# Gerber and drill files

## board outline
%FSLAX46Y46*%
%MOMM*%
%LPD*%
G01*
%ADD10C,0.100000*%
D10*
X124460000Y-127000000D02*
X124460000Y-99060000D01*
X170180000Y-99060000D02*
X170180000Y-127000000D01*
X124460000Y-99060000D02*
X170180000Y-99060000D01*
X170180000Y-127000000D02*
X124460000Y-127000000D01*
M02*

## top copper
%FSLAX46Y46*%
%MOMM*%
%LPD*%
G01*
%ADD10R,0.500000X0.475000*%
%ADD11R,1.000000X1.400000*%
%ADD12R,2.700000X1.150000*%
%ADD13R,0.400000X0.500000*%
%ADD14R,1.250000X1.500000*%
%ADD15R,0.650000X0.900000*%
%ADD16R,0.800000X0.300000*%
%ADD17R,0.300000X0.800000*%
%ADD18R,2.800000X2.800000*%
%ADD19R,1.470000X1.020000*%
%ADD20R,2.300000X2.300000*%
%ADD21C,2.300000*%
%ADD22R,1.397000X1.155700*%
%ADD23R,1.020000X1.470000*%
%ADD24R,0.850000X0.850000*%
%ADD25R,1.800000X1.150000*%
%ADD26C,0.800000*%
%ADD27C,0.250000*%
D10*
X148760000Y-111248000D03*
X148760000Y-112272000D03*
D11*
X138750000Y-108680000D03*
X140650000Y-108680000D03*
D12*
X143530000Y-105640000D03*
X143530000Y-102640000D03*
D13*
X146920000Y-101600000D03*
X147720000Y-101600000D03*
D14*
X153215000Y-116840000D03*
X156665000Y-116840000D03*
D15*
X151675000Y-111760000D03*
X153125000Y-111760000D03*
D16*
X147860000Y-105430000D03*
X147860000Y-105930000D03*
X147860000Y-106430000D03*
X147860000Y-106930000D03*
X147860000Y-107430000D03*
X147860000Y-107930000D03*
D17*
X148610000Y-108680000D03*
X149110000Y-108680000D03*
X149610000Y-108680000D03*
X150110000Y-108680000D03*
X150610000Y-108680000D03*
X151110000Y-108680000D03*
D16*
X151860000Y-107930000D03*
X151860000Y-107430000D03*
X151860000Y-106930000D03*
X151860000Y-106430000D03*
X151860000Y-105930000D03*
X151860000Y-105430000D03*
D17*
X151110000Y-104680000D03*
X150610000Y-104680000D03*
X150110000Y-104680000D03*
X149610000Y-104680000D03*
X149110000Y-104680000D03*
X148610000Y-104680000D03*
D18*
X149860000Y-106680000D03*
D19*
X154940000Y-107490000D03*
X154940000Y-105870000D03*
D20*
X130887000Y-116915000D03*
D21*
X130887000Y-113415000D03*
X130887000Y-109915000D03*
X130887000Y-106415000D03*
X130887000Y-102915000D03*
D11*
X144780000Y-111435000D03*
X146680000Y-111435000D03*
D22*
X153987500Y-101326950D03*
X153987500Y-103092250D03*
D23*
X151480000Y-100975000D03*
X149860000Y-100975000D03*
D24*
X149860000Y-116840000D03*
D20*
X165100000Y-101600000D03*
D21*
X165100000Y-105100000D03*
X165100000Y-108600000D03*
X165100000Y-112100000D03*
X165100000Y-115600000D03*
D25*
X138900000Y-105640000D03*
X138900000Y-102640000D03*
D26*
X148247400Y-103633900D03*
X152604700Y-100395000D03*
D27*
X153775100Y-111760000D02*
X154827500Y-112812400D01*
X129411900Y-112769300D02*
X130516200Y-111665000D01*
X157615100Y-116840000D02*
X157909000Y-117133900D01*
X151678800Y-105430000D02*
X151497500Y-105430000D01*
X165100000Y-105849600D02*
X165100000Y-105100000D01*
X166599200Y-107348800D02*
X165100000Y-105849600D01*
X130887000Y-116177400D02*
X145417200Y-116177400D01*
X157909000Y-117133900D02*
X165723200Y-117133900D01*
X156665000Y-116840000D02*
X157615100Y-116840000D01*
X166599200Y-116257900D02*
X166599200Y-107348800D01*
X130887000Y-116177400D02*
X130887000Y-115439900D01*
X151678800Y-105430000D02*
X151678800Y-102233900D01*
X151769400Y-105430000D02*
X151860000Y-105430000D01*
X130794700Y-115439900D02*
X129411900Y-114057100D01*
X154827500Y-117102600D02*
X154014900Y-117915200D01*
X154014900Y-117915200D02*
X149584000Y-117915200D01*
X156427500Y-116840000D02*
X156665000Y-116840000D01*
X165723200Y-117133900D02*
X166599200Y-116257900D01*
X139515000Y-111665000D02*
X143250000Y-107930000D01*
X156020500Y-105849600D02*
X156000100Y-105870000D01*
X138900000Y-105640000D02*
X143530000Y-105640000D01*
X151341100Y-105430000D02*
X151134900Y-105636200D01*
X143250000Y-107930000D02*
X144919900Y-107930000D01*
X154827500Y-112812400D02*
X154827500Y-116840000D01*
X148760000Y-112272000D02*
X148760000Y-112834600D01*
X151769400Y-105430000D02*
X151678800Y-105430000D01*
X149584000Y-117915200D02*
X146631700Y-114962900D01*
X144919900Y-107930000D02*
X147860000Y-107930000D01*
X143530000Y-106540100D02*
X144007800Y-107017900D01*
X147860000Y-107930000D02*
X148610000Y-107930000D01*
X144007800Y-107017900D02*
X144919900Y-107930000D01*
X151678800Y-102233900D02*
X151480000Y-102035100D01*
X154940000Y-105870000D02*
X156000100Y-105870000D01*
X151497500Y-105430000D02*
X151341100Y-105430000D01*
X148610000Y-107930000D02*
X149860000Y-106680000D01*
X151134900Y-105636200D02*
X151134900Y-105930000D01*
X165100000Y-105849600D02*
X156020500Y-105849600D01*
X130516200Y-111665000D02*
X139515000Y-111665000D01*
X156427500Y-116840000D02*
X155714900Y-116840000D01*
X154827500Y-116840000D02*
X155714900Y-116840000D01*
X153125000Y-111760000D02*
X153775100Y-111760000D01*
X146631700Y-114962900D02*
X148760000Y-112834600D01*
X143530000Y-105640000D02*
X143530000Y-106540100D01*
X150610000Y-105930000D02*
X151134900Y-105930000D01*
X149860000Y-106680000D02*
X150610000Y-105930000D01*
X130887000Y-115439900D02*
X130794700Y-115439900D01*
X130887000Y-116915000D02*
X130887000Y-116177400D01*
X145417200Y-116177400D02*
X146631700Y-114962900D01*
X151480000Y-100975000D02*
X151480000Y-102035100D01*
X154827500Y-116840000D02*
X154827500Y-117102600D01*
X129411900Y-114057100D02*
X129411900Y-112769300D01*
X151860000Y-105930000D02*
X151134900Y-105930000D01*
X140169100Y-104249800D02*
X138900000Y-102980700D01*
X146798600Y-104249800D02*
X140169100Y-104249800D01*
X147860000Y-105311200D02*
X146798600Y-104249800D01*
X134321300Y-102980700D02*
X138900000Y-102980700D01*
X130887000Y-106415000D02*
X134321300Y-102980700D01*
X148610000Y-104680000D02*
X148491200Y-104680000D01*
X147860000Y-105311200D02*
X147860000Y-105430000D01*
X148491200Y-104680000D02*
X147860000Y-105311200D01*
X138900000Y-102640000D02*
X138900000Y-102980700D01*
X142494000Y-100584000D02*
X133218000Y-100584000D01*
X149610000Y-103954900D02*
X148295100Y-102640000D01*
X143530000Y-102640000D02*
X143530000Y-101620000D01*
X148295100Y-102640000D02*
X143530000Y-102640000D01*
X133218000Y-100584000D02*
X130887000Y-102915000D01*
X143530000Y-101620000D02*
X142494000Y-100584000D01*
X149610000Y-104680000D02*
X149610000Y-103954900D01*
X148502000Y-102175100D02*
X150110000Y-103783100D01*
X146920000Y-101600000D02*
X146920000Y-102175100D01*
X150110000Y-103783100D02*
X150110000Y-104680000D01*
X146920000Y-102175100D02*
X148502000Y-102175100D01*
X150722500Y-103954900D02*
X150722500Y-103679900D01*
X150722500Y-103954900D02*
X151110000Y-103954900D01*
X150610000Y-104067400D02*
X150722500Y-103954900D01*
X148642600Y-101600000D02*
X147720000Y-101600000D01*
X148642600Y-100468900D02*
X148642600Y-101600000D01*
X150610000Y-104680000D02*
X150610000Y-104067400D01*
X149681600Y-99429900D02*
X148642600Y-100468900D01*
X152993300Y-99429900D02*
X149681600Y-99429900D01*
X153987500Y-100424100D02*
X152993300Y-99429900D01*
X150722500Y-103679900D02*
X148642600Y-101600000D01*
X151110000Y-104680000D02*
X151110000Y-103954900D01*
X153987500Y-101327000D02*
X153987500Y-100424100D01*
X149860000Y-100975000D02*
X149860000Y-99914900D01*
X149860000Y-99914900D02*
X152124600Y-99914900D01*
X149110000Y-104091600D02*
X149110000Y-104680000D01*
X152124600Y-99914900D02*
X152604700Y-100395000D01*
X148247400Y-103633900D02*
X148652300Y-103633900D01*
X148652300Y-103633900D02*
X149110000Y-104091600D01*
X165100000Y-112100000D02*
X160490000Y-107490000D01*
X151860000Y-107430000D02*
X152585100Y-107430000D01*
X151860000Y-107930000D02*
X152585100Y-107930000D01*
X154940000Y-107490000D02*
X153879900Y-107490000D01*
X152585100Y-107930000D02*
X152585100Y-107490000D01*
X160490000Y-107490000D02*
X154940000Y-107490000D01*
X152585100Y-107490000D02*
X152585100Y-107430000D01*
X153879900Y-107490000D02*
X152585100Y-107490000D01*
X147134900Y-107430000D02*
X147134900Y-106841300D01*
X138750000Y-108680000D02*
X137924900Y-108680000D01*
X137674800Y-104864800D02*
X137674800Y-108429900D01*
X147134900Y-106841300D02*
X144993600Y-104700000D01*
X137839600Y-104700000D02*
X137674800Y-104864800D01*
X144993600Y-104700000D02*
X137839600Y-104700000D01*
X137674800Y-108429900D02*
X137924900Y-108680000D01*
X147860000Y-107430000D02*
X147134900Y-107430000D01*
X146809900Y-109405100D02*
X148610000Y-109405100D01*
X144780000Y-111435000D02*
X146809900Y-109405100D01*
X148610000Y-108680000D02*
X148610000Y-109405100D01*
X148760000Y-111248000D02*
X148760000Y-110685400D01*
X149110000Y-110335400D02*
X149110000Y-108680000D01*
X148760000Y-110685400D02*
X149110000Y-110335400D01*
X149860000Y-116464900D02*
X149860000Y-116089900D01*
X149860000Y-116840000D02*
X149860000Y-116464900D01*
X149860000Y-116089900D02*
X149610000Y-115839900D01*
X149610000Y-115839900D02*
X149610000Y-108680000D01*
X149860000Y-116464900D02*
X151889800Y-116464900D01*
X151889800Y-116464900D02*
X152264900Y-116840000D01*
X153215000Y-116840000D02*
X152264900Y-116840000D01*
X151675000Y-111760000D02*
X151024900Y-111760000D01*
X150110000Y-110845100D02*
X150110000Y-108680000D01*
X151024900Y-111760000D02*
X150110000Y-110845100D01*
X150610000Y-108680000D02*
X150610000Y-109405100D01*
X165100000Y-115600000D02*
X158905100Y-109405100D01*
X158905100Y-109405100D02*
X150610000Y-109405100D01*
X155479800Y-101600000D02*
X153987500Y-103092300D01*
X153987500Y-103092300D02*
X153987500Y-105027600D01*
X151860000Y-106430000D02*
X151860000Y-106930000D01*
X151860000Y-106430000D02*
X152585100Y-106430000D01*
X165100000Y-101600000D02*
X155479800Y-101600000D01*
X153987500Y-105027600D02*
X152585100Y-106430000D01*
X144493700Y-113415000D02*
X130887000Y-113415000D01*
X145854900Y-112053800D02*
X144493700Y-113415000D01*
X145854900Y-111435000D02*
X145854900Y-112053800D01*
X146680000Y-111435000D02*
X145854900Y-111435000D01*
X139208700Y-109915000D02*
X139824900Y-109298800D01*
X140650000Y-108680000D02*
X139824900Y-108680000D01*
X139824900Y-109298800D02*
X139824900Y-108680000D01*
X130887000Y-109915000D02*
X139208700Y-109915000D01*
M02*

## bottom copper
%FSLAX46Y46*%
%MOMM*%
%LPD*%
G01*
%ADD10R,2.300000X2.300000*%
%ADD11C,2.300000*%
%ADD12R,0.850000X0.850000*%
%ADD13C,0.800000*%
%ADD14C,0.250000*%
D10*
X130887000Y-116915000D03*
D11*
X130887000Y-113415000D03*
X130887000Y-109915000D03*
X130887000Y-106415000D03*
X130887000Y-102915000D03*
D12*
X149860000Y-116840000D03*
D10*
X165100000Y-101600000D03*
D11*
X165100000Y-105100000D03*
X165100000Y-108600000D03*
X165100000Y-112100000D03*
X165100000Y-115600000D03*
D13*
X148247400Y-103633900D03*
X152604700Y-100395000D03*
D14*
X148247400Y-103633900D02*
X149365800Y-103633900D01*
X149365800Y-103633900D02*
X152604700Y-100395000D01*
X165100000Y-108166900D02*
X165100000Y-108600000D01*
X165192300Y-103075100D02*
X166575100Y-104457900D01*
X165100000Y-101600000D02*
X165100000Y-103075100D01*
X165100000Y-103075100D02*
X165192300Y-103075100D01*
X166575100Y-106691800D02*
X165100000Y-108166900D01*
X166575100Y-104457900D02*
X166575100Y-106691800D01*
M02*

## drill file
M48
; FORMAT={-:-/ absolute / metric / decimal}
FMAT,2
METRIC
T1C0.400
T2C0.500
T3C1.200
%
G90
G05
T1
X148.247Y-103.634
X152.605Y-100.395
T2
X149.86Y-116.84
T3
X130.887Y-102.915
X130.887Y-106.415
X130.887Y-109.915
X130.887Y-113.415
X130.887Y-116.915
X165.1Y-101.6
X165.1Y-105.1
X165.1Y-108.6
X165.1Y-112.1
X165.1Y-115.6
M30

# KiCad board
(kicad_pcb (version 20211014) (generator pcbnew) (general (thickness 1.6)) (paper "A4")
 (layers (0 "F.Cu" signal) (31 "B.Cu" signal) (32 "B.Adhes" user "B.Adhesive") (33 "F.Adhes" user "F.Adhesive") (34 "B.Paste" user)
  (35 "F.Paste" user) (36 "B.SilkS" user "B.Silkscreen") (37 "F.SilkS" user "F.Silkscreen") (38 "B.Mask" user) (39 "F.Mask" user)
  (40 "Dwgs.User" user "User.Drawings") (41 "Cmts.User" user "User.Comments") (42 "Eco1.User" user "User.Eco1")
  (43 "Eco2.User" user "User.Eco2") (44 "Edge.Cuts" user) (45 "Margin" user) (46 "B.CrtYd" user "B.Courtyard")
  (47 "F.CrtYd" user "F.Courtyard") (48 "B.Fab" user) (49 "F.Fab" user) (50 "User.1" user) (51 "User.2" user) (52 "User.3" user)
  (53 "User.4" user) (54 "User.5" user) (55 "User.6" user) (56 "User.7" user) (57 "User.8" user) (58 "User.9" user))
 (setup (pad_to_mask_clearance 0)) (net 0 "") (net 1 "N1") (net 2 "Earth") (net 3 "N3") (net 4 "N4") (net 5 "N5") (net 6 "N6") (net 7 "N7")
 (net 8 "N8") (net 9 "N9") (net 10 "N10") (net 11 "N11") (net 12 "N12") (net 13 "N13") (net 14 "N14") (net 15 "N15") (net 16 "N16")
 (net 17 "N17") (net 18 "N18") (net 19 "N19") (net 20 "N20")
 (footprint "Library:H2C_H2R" (layer "F.Cu") (at 148.76 111.76 -90)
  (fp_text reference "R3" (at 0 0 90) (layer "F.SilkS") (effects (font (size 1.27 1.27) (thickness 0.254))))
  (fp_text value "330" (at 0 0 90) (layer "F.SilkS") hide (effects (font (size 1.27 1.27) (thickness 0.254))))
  (pad "1" smd rect locked (at -0.512 0 270) (size 0.475 0.5) (layers "F.Cu" "F.Paste" "F.Mask") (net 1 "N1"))
  (pad "2" smd rect locked (at 0.512 0 270) (size 0.475 0.5) (layers "F.Cu" "F.Paste" "F.Mask") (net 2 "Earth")))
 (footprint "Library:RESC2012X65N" (layer "F.Cu") (at 139.7 108.68)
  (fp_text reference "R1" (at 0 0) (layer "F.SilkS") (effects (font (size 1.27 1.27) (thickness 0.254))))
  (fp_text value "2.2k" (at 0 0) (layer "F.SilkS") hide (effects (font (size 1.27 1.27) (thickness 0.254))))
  (pad "1" smd rect (at -0.95 0) (size 1 1.4) (layers "F.Cu" "F.Paste" "F.Mask") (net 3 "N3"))
  (pad "2" smd rect (at 0.95 0) (size 1 1.4) (layers "F.Cu" "F.Paste" "F.Mask") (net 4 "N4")))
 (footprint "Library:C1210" (layer "F.Cu") (at 143.53 104.14 90)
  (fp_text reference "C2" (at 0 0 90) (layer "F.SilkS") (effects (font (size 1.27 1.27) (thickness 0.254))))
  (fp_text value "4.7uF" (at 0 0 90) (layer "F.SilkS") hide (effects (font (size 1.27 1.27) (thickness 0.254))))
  (pad "1" smd rect (at -1.5 0 90) (size 1.15 2.7) (layers "F.Cu" "F.Paste" "F.Mask") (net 2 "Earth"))
  (pad "2" smd rect (at 1.5 0 90) (size 1.15 2.7) (layers "F.Cu" "F.Paste" "F.Mask") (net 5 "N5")))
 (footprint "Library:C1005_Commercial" (layer "F.Cu") (at 147.32 101.6)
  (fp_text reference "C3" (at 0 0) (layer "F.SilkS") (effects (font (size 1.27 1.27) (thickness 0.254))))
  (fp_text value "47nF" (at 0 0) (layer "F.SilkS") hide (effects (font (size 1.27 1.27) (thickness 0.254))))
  (pad "1" smd rect (at -0.4 0) (size 0.4 0.5) (layers "F.Cu" "F.Paste" "F.Mask") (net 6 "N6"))
  (pad "2" smd rect (at 0.4 0) (size 0.4 0.5) (layers "F.Cu" "F.Paste" "F.Mask") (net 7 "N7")))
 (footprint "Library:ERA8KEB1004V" (layer "F.Cu") (at 154.94 116.84)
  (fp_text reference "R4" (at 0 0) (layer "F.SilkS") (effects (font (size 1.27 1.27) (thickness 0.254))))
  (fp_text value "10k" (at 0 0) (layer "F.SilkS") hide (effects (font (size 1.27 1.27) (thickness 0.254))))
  (pad "1" smd rect locked (at -1.725 0) (size 1.25 1.5) (layers "F.Cu" "F.Paste" "F.Mask") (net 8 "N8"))
  (pad "2" smd rect locked (at 1.725 0) (size 1.25 1.5) (layers "F.Cu" "F.Paste" "F.Mask") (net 2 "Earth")))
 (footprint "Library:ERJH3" (layer "F.Cu") (at 152.4 111.76)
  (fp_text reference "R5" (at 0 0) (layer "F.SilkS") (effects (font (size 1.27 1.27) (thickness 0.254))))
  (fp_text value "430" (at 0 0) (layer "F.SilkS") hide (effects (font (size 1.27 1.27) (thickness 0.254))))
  (pad "1" smd rect locked (at -0.725 0) (size 0.65 0.9) (layers "F.Cu" "F.Paste" "F.Mask") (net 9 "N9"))
  (pad "2" smd rect locked (at 0.725 0) (size 0.65 0.9) (layers "F.Cu" "F.Paste" "F.Mask") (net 2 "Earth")))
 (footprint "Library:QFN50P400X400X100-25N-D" (layer "F.Cu") (at 149.86 106.68)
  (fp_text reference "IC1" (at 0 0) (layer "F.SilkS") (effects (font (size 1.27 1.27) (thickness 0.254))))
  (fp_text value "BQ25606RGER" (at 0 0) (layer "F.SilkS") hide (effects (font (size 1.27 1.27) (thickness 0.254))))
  (pad "1" smd rect (at -2 -1.25 90) (size 0.3 0.8) (layers "F.Cu" "F.Paste" "F.Mask") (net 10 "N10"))
  (pad "2" smd rect (at -2 -0.75 90) (size 0.3 0.8) (layers "F.Cu" "F.Paste" "F.Mask") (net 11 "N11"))
  (pad "3" smd rect (at -2 -0.25 90) (size 0.3 0.8) (layers "F.Cu" "F.Paste" "F.Mask") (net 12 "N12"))
  (pad "4" smd rect (at -2 0.25 90) (size 0.3 0.8) (layers "F.Cu" "F.Paste" "F.Mask") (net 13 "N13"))
  (pad "5" smd rect (at -2 0.75 90) (size 0.3 0.8) (layers "F.Cu" "F.Paste" "F.Mask") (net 3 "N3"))
  (pad "6" smd rect (at -2 1.25 90) (size 0.3 0.8) (layers "F.Cu" "F.Paste" "F.Mask") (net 2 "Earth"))
  (pad "7" smd rect (at -1.25 2) (size 0.3 0.8) (layers "F.Cu" "F.Paste" "F.Mask") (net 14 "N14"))
  (pad "8" smd rect (at -0.75 2) (size 0.3 0.8) (layers "F.Cu" "F.Paste" "F.Mask") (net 1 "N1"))
  (pad "9" smd rect (at -0.25 2) (size 0.3 0.8) (layers "F.Cu" "F.Paste" "F.Mask") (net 8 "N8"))
  (pad "10" smd rect (at 0.25 2) (size 0.3 0.8) (layers "F.Cu" "F.Paste" "F.Mask") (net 9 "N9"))
  (pad "11" smd rect (at 0.75 2) (size 0.3 0.8) (layers "F.Cu" "F.Paste" "F.Mask") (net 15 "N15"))
  (pad "12" smd rect (at 1.25 2) (size 0.3 0.8) (layers "F.Cu" "F.Paste" "F.Mask") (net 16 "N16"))
  (pad "13" smd rect (at 2 1.25 90) (size 0.3 0.8) (layers "F.Cu" "F.Paste" "F.Mask") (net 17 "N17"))
  (pad "14" smd rect (at 2 0.75 90) (size 0.3 0.8) (layers "F.Cu" "F.Paste" "F.Mask") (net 17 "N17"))
  (pad "15" smd rect (at 2 0.25 90) (size 0.3 0.8) (layers "F.Cu" "F.Paste" "F.Mask") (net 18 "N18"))
  (pad "16" smd rect (at 2 -0.25 90) (size 0.3 0.8) (layers "F.Cu" "F.Paste" "F.Mask") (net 18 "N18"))
  (pad "17" smd rect (at 2 -0.75 90) (size 0.3 0.8) (layers "F.Cu" "F.Paste" "F.Mask") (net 2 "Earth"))
  (pad "18" smd rect (at 2 -1.25 90) (size 0.3 0.8) (layers "F.Cu" "F.Paste" "F.Mask") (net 2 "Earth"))
  (pad "19" smd rect (at 1.25 -2) (size 0.3 0.8) (layers "F.Cu" "F.Paste" "F.Mask") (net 7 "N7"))
  (pad "20" smd rect (at 0.75 -2) (size 0.3 0.8) (layers "F.Cu" "F.Paste" "F.Mask") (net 7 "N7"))
  (pad "21" smd rect (at 0.25 -2) (size 0.3 0.8) (layers "F.Cu" "F.Paste" "F.Mask") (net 6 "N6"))
  (pad "22" smd rect (at -0.25 -2) (size 0.3 0.8) (layers "F.Cu" "F.Paste" "F.Mask") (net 5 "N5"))
  (pad "23" smd rect (at -0.75 -2) (size 0.3 0.8) (layers "F.Cu" "F.Paste" "F.Mask") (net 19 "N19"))
  (pad "24" smd rect (at -1.25 -2) (size 0.3 0.8) (layers "F.Cu" "F.Paste" "F.Mask") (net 10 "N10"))
  (pad "25" smd rect (at 0 0) (size 2.8 2.8) (layers "F.Cu" "F.Paste" "F.Mask") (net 2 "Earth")))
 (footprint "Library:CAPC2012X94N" (layer "F.Cu") (at 154.94 106.68 90)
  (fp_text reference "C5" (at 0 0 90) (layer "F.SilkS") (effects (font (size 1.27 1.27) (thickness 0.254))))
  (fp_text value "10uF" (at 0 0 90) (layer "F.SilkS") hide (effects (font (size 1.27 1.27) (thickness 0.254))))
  (pad "1" smd rect (at -0.81 0 90) (size 1.02 1.47) (layers "F.Cu" "F.Paste" "F.Mask") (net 17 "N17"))
  (pad "2" smd rect (at 0.81 0 90) (size 1.02 1.47) (layers "F.Cu" "F.Paste" "F.Mask") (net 2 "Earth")))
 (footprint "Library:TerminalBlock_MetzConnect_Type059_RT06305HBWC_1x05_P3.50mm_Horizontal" (layer "F.Cu") (at 130.887 116.915 90)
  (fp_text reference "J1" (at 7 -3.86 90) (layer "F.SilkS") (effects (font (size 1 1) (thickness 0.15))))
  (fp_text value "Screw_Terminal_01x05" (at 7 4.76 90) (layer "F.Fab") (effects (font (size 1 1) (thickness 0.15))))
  (pad "1" thru_hole rect (at 0 0 90) (size 2.3 2.3) (drill 1.2) (layers *.Cu *.Mask) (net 2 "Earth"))
  (pad "2" thru_hole circle (at 3.5 0 90) (size 2.3 2.3) (drill 1.2) (layers *.Cu *.Mask) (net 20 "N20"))
  (pad "3" thru_hole circle (at 7 0 90) (size 2.3 2.3) (drill 1.2) (layers *.Cu *.Mask) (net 4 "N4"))
  (pad "4" thru_hole circle (at 10.5 0 90) (size 2.3 2.3) (drill 1.2) (layers *.Cu *.Mask) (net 10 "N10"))
  (pad "5" thru_hole circle (at 14 0 90) (size 2.3 2.3) (drill 1.2) (layers *.Cu *.Mask) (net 5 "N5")))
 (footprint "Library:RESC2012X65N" (layer "F.Cu") (at 145.73 111.435)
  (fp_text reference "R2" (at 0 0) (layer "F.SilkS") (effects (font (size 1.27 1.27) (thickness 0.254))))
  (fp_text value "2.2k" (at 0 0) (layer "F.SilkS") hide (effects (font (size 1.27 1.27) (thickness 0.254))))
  (pad "1" smd rect (at -0.95 0) (size 1 1.4) (layers "F.Cu" "F.Paste" "F.Mask") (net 14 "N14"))
  (pad "2" smd rect (at 0.95 0) (size 1 1.4) (layers "F.Cu" "F.Paste" "F.Mask") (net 20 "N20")))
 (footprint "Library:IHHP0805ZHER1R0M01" (layer "F.Cu") (at 153.9875 102.2096 -90)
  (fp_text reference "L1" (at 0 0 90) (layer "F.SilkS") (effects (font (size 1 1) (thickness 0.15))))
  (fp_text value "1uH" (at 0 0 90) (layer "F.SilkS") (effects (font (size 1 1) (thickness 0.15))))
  (pad "1" smd rect (at -0.88265 0 270) (size 1.1557 1.397) (layers "F.Cu" "F.Paste" "F.Mask") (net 7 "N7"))
  (pad "2" smd rect (at 0.88265 0 270) (size 1.1557 1.397) (layers "F.Cu" "F.Paste" "F.Mask") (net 18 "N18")))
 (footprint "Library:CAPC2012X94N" (layer "F.Cu") (at 150.67 100.975 180)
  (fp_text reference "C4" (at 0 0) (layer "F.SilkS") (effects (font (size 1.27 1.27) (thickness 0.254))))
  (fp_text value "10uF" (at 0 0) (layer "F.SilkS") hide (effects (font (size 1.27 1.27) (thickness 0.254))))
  (pad "1" smd rect (at -0.81 0 180) (size 1.02 1.47) (layers "F.Cu" "F.Paste" "F.Mask") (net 2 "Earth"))
  (pad "2" smd rect (at 0.81 0 180) (size 1.02 1.47) (layers "F.Cu" "F.Paste" "F.Mask") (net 19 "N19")))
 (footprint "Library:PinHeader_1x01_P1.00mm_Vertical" (layer "F.Cu") (at 149.86 116.84)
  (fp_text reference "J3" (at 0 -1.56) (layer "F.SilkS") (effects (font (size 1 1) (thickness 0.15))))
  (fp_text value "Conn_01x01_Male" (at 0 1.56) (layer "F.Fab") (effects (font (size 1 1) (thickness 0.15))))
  (pad "1" thru_hole rect (at 0 0) (size 0.85 0.85) (drill 0.5) (layers *.Cu *.Mask) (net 8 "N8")))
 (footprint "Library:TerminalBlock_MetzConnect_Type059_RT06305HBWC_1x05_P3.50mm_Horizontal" (layer "F.Cu") (at 165.1 101.6 -90)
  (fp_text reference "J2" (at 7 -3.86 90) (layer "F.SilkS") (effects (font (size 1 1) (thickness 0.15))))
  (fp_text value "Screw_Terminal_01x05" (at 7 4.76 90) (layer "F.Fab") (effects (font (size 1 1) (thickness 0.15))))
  (pad "1" thru_hole rect (at 0 0 270) (size 2.3 2.3) (drill 1.2) (layers *.Cu *.Mask) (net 18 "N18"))
  (pad "2" thru_hole circle (at 3.5 0 270) (size 2.3 2.3) (drill 1.2) (layers *.Cu *.Mask) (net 2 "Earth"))
  (pad "3" thru_hole circle (at 7 0 270) (size 2.3 2.3) (drill 1.2) (layers *.Cu *.Mask) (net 18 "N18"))
  (pad "4" thru_hole circle (at 10.5 0 270) (size 2.3 2.3) (drill 1.2) (layers *.Cu *.Mask) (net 17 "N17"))
  (pad "5" thru_hole circle (at 14 0 270) (size 2.3 2.3) (drill 1.2) (layers *.Cu *.Mask) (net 15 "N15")))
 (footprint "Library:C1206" (layer "F.Cu") (at 138.9 104.14 90)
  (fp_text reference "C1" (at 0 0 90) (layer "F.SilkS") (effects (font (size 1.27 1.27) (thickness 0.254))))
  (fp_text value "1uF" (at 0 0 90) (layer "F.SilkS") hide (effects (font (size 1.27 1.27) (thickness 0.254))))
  (pad "1" smd rect (at -1.5 0 90) (size 1.15 1.8) (layers "F.Cu" "F.Paste" "F.Mask") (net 2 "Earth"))
  (pad "2" smd rect (at 1.5 0 90) (size 1.15 1.8) (layers "F.Cu" "F.Paste" "F.Mask") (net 10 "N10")))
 (gr_line (start 124.46 127) (end 124.46 99.06) (layer "Edge.Cuts") (width 0.1))
 (gr_line (start 170.18 99.06) (end 170.18 127) (layer "Edge.Cuts") (width 0.1))
 (gr_line (start 124.46 99.06) (end 170.18 99.06) (layer "Edge.Cuts") (width 0.1))
 (gr_line (start 170.18 127) (end 124.46 127) (layer "Edge.Cuts") (width 0.1))
 (segment (start 153.7751 111.76) (end 154.8275 112.8124) (width 0.25) (layer "F.Cu") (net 2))
 (segment (start 129.4119 112.7693) (end 130.5162 111.665) (width 0.25) (layer "F.Cu") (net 2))
 (segment (start 157.6151 116.84) (end 157.909 117.1339) (width 0.25) (layer "F.Cu") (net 2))
 (segment (start 151.6788 105.43) (end 151.4975 105.43) (width 0.25) (layer "F.Cu") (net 2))
 (segment (start 165.1 105.8496) (end 165.1 105.1) (width 0.25) (layer "F.Cu") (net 2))
 (segment (start 166.5992 107.3488) (end 165.1 105.8496) (width 0.25) (layer "F.Cu") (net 2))
 (segment (start 130.887 116.1774) (end 145.4172 116.1774) (width 0.25) (layer "F.Cu") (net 2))
 (segment (start 157.909 117.1339) (end 165.7232 117.1339) (width 0.25) (layer "F.Cu") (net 2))
 (segment (start 156.665 116.84) (end 157.6151 116.84) (width 0.25) (layer "F.Cu") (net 2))
 (segment (start 166.5992 116.2579) (end 166.5992 107.3488) (width 0.25) (layer "F.Cu") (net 2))
 (segment (start 130.887 116.1774) (end 130.887 115.4399) (width 0.25) (layer "F.Cu") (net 2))
 (segment (start 151.6788 105.43) (end 151.6788 102.2339) (width 0.25) (layer "F.Cu") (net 2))
 (segment (start 151.7694 105.43) (end 151.86 105.43) (width 0.25) (layer "F.Cu") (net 2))
 (segment (start 130.7947 115.4399) (end 129.4119 114.0571) (width 0.25) (layer "F.Cu") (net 2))
 (segment (start 154.8275 117.1026) (end 154.0149 117.9152) (width 0.25) (layer "F.Cu") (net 2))
 (segment (start 154.0149 117.9152) (end 149.584 117.9152) (width 0.25) (layer "F.Cu") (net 2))
 (segment (start 156.4275 116.84) (end 156.665 116.84) (width 0.25) (layer "F.Cu") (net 2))
 (segment (start 165.7232 117.1339) (end 166.5992 116.2579) (width 0.25) (layer "F.Cu") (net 2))
 (segment (start 139.515 111.665) (end 143.25 107.93) (width 0.25) (layer "F.Cu") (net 2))
 (segment (start 156.0205 105.8496) (end 156.0001 105.87) (width 0.25) (layer "F.Cu") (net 2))
 (segment (start 138.9 105.64) (end 143.53 105.64) (width 0.25) (layer "F.Cu") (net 2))
 (segment (start 151.3411 105.43) (end 151.1349 105.6362) (width 0.25) (layer "F.Cu") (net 2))
 (segment (start 143.25 107.93) (end 144.9199 107.93) (width 0.25) (layer "F.Cu") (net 2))
 (segment (start 154.8275 112.8124) (end 154.8275 116.84) (width 0.25) (layer "F.Cu") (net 2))
 (segment (start 148.76 112.272) (end 148.76 112.8346) (width 0.25) (layer "F.Cu") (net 2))
 (segment (start 151.7694 105.43) (end 151.6788 105.43) (width 0.25) (layer "F.Cu") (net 2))
 (segment (start 149.584 117.9152) (end 146.6317 114.9629) (width 0.25) (layer "F.Cu") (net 2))
 (segment (start 144.9199 107.93) (end 147.86 107.93) (width 0.25) (layer "F.Cu") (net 2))
 (segment (start 143.53 106.5401) (end 144.0078 107.0179) (width 0.25) (layer "F.Cu") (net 2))
 (segment (start 147.86 107.93) (end 148.61 107.93) (width 0.25) (layer "F.Cu") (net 2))
 (segment (start 144.0078 107.0179) (end 144.9199 107.93) (width 0.25) (layer "F.Cu") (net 2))
 (segment (start 151.6788 102.2339) (end 151.48 102.0351) (width 0.25) (layer "F.Cu") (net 2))
 (segment (start 154.94 105.87) (end 156.0001 105.87) (width 0.25) (layer "F.Cu") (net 2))
 (segment (start 151.4975 105.43) (end 151.3411 105.43) (width 0.25) (layer "F.Cu") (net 2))
 (segment (start 148.61 107.93) (end 149.86 106.68) (width 0.25) (layer "F.Cu") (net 2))
 (segment (start 151.1349 105.6362) (end 151.1349 105.93) (width 0.25) (layer "F.Cu") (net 2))
 (segment (start 165.1 105.8496) (end 156.0205 105.8496) (width 0.25) (layer "F.Cu") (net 2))
 (segment (start 130.5162 111.665) (end 139.515 111.665) (width 0.25) (layer "F.Cu") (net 2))
 (segment (start 156.4275 116.84) (end 155.7149 116.84) (width 0.25) (layer "F.Cu") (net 2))
 (segment (start 154.8275 116.84) (end 155.7149 116.84) (width 0.25) (layer "F.Cu") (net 2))
 (segment (start 153.125 111.76) (end 153.7751 111.76) (width 0.25) (layer "F.Cu") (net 2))
 (segment (start 146.6317 114.9629) (end 148.76 112.8346) (width 0.25) (layer "F.Cu") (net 2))
 (segment (start 143.53 105.64) (end 143.53 106.5401) (width 0.25) (layer "F.Cu") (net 2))
 (segment (start 150.61 105.93) (end 151.1349 105.93) (width 0.25) (layer "F.Cu") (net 2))
 (segment (start 149.86 106.68) (end 150.61 105.93) (width 0.25) (layer "F.Cu") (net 2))
 (segment (start 130.887 115.4399) (end 130.7947 115.4399) (width 0.25) (layer "F.Cu") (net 2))
 (segment (start 130.887 116.915) (end 130.887 116.1774) (width 0.25) (layer "F.Cu") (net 2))
 (segment (start 145.4172 116.1774) (end 146.6317 114.9629) (width 0.25) (layer "F.Cu") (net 2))
 (segment (start 151.48 100.975) (end 151.48 102.0351) (width 0.25) (layer "F.Cu") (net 2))
 (segment (start 154.8275 116.84) (end 154.8275 117.1026) (width 0.25) (layer "F.Cu") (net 2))
 (segment (start 129.4119 114.0571) (end 129.4119 112.7693) (width 0.25) (layer "F.Cu") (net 2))
 (segment (start 151.86 105.93) (end 151.1349 105.93) (width 0.25) (layer "F.Cu") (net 2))
 (segment (start 140.1691 104.2498) (end 138.9 102.9807) (width 0.25) (layer "F.Cu") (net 10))
 (segment (start 146.7986 104.2498) (end 140.1691 104.2498) (width 0.25) (layer "F.Cu") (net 10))
 (segment (start 147.86 105.3112) (end 146.7986 104.2498) (width 0.25) (layer "F.Cu") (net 10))
 (segment (start 134.3213 102.9807) (end 138.9 102.9807) (width 0.25) (layer "F.Cu") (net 10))
 (segment (start 130.887 106.415) (end 134.3213 102.9807) (width 0.25) (layer "F.Cu") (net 10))
 (segment (start 148.61 104.68) (end 148.4912 104.68) (width 0.25) (layer "F.Cu") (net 10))
 (segment (start 147.86 105.3112) (end 147.86 105.43) (width 0.25) (layer "F.Cu") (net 10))
 (segment (start 148.4912 104.68) (end 147.86 105.3112) (width 0.25) (layer "F.Cu") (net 10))
 (segment (start 138.9 102.64) (end 138.9 102.9807) (width 0.25) (layer "F.Cu") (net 10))
 (segment (start 142.494 100.584) (end 133.218 100.584) (width 0.25) (layer "F.Cu") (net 5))
 (segment (start 149.61 103.9549) (end 148.2951 102.64) (width 0.25) (layer "F.Cu") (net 5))
 (segment (start 143.53 102.64) (end 143.53 101.62) (width 0.25) (layer "F.Cu") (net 5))
 (segment (start 148.2951 102.64) (end 143.53 102.64) (width 0.25) (layer "F.Cu") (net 5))
 (segment (start 133.218 100.584) (end 130.887 102.915) (width 0.25) (layer "F.Cu") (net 5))
 (segment (start 143.53 101.62) (end 142.494 100.584) (width 0.25) (layer "F.Cu") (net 5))
 (segment (start 149.61 104.68) (end 149.61 103.9549) (width 0.25) (layer "F.Cu") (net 5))
 (segment (start 148.502 102.1751) (end 150.11 103.7831) (width 0.25) (layer "F.Cu") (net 6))
 (segment (start 146.92 101.6) (end 146.92 102.1751) (width 0.25) (layer "F.Cu") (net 6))
 (segment (start 150.11 103.7831) (end 150.11 104.68) (width 0.25) (layer "F.Cu") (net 6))
 (segment (start 146.92 102.1751) (end 148.502 102.1751) (width 0.25) (layer "F.Cu") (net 6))
 (segment (start 150.7225 103.9549) (end 150.7225 103.6799) (width 0.25) (layer "F.Cu") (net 7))
 (segment (start 150.7225 103.9549) (end 151.11 103.9549) (width 0.25) (layer "F.Cu") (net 7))
 (segment (start 150.61 104.0674) (end 150.7225 103.9549) (width 0.25) (layer "F.Cu") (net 7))
 (segment (start 148.6426 101.6) (end 147.72 101.6) (width 0.25) (layer "F.Cu") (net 7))
 (segment (start 148.6426 100.4689) (end 148.6426 101.6) (width 0.25) (layer "F.Cu") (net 7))
 (segment (start 150.61 104.68) (end 150.61 104.0674) (width 0.25) (layer "F.Cu") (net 7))
 (segment (start 149.6816 99.4299) (end 148.6426 100.4689) (width 0.25) (layer "F.Cu") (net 7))
 (segment (start 152.9933 99.4299) (end 149.6816 99.4299) (width 0.25) (layer "F.Cu") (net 7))
 (segment (start 153.9875 100.4241) (end 152.9933 99.4299) (width 0.25) (layer "F.Cu") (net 7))
 (segment (start 150.7225 103.6799) (end 148.6426 101.6) (width 0.25) (layer "F.Cu") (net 7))
 (segment (start 151.11 104.68) (end 151.11 103.9549) (width 0.25) (layer "F.Cu") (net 7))
 (segment (start 153.9875 101.327) (end 153.9875 100.4241) (width 0.25) (layer "F.Cu") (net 7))
 (segment (start 149.86 100.975) (end 149.86 99.9149) (width 0.25) (layer "F.Cu") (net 19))
 (segment (start 149.86 99.9149) (end 152.1246 99.9149) (width 0.25) (layer "F.Cu") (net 19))
 (segment (start 149.11 104.0916) (end 149.11 104.68) (width 0.25) (layer "F.Cu") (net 19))
 (segment (start 152.1246 99.9149) (end 152.6047 100.395) (width 0.25) (layer "F.Cu") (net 19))
 (segment (start 148.2474 103.6339) (end 148.6523 103.6339) (width 0.25) (layer "F.Cu") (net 19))
 (segment (start 148.6523 103.6339) (end 149.11 104.0916) (width 0.25) (layer "F.Cu") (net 19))
 (via (at 148.2474 103.6339) (size 0.8) (drill 0.4) (layers "F.Cu" "B.Cu") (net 19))
 (via (at 152.6047 100.395) (size 0.8) (drill 0.4) (layers "F.Cu" "B.Cu") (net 19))
 (segment (start 148.2474 103.6339) (end 149.3658 103.6339) (width 0.25) (layer "B.Cu") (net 19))
 (segment (start 149.3658 103.6339) (end 152.6047 100.395) (width 0.25) (layer "B.Cu") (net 19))
 (segment (start 165.1 112.1) (end 160.49 107.49) (width 0.25) (layer "F.Cu") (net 17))
 (segment (start 151.86 107.43) (end 152.5851 107.43) (width 0.25) (layer "F.Cu") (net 17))
 (segment (start 151.86 107.93) (end 152.5851 107.93) (width 0.25) (layer "F.Cu") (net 17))
 (segment (start 154.94 107.49) (end 153.8799 107.49) (width 0.25) (layer "F.Cu") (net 17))
 (segment (start 152.5851 107.93) (end 152.5851 107.49) (width 0.25) (layer "F.Cu") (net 17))
 (segment (start 160.49 107.49) (end 154.94 107.49) (width 0.25) (layer "F.Cu") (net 17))
 (segment (start 152.5851 107.49) (end 152.5851 107.43) (width 0.25) (layer "F.Cu") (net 17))
 (segment (start 153.8799 107.49) (end 152.5851 107.49) (width 0.25) (layer "F.Cu") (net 17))
 (segment (start 147.1349 107.43) (end 147.1349 106.8413) (width 0.25) (layer "F.Cu") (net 3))
 (segment (start 138.75 108.68) (end 137.9249 108.68) (width 0.25) (layer "F.Cu") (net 3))
 (segment (start 137.6748 104.8648) (end 137.6748 108.4299) (width 0.25) (layer "F.Cu") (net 3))
 (segment (start 147.1349 106.8413) (end 144.9936 104.7) (width 0.25) (layer "F.Cu") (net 3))
 (segment (start 137.8396 104.7) (end 137.6748 104.8648) (width 0.25) (layer "F.Cu") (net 3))
 (segment (start 144.9936 104.7) (end 137.8396 104.7) (width 0.25) (layer "F.Cu") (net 3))
 (segment (start 137.6748 108.4299) (end 137.9249 108.68) (width 0.25) (layer "F.Cu") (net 3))
 (segment (start 147.86 107.43) (end 147.1349 107.43) (width 0.25) (layer "F.Cu") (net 3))
 (segment (start 146.8099 109.4051) (end 148.61 109.4051) (width 0.25) (layer "F.Cu") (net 14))
 (segment (start 144.78 111.435) (end 146.8099 109.4051) (width 0.25) (layer "F.Cu") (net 14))
 (segment (start 148.61 108.68) (end 148.61 109.4051) (width 0.25) (layer "F.Cu") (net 14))
 (segment (start 148.76 111.248) (end 148.76 110.6854) (width 0.25) (layer "F.Cu") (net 1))
 (segment (start 149.11 110.3354) (end 149.11 108.68) (width 0.25) (layer "F.Cu") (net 1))
 (segment (start 148.76 110.6854) (end 149.11 110.3354) (width 0.25) (layer "F.Cu") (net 1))
 (segment (start 149.86 116.4649) (end 149.86 116.0899) (width 0.25) (layer "F.Cu") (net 8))
 (segment (start 149.86 116.84) (end 149.86 116.4649) (width 0.25) (layer "F.Cu") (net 8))
 (segment (start 149.86 116.0899) (end 149.61 115.8399) (width 0.25) (layer "F.Cu") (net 8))
 (segment (start 149.61 115.8399) (end 149.61 108.68) (width 0.25) (layer "F.Cu") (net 8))
 (segment (start 149.86 116.4649) (end 151.8898 116.4649) (width 0.25) (layer "F.Cu") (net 8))
 (segment (start 151.8898 116.4649) (end 152.2649 116.84) (width 0.25) (layer "F.Cu") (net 8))
 (segment (start 153.215 116.84) (end 152.2649 116.84) (width 0.25) (layer "F.Cu") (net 8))
 (segment (start 151.675 111.76) (end 151.0249 111.76) (width 0.25) (layer "F.Cu") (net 9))
 (segment (start 150.11 110.8451) (end 150.11 108.68) (width 0.25) (layer "F.Cu") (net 9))
 (segment (start 151.0249 111.76) (end 150.11 110.8451) (width 0.25) (layer "F.Cu") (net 9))
 (segment (start 150.61 108.68) (end 150.61 109.4051) (width 0.25) (layer "F.Cu") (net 15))
 (segment (start 165.1 115.6) (end 158.9051 109.4051) (width 0.25) (layer "F.Cu") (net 15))
 (segment (start 158.9051 109.4051) (end 150.61 109.4051) (width 0.25) (layer "F.Cu") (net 15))
 (segment (start 155.4798 101.6) (end 153.9875 103.0923) (width 0.25) (layer "F.Cu") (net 18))
 (segment (start 153.9875 103.0923) (end 153.9875 105.0276) (width 0.25) (layer "F.Cu") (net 18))
 (segment (start 151.86 106.43) (end 151.86 106.93) (width 0.25) (layer "F.Cu") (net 18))
 (segment (start 151.86 106.43) (end 152.5851 106.43) (width 0.25) (layer "F.Cu") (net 18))
 (segment (start 165.1 101.6) (end 155.4798 101.6) (width 0.25) (layer "F.Cu") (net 18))
 (segment (start 153.9875 105.0276) (end 152.5851 106.43) (width 0.25) (layer "F.Cu") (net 18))
 (segment (start 165.1 108.1669) (end 165.1 108.6) (width 0.25) (layer "B.Cu") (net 18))
 (segment (start 165.1923 103.0751) (end 166.5751 104.4579) (width 0.25) (layer "B.Cu") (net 18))
 (segment (start 165.1 101.6) (end 165.1 103.0751) (width 0.25) (layer "B.Cu") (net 18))
 (segment (start 165.1 103.0751) (end 165.1923 103.0751) (width 0.25) (layer "B.Cu") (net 18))
 (segment (start 166.5751 106.6918) (end 165.1 108.1669) (width 0.25) (layer "B.Cu") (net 18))
 (segment (start 166.5751 104.4579) (end 166.5751 106.6918) (width 0.25) (layer "B.Cu") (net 18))
 (segment (start 144.4937 113.415) (end 130.887 113.415) (width 0.25) (layer "F.Cu") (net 20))
 (segment (start 145.8549 112.0538) (end 144.4937 113.415) (width 0.25) (layer "F.Cu") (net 20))
 (segment (start 145.8549 111.435) (end 145.8549 112.0538) (width 0.25) (layer "F.Cu") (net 20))
 (segment (start 146.68 111.435) (end 145.8549 111.435) (width 0.25) (layer "F.Cu") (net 20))
 (segment (start 139.2087 109.915) (end 139.8249 109.2988) (width 0.25) (layer "F.Cu") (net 4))
 (segment (start 140.65 108.68) (end 139.8249 108.68) (width 0.25) (layer "F.Cu") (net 4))
 (segment (start 139.8249 109.2988) (end 139.8249 108.68) (width 0.25) (layer "F.Cu") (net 4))
 (segment (start 130.887 109.915) (end 139.2087 109.915) (width 0.25) (layer "F.Cu") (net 4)))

